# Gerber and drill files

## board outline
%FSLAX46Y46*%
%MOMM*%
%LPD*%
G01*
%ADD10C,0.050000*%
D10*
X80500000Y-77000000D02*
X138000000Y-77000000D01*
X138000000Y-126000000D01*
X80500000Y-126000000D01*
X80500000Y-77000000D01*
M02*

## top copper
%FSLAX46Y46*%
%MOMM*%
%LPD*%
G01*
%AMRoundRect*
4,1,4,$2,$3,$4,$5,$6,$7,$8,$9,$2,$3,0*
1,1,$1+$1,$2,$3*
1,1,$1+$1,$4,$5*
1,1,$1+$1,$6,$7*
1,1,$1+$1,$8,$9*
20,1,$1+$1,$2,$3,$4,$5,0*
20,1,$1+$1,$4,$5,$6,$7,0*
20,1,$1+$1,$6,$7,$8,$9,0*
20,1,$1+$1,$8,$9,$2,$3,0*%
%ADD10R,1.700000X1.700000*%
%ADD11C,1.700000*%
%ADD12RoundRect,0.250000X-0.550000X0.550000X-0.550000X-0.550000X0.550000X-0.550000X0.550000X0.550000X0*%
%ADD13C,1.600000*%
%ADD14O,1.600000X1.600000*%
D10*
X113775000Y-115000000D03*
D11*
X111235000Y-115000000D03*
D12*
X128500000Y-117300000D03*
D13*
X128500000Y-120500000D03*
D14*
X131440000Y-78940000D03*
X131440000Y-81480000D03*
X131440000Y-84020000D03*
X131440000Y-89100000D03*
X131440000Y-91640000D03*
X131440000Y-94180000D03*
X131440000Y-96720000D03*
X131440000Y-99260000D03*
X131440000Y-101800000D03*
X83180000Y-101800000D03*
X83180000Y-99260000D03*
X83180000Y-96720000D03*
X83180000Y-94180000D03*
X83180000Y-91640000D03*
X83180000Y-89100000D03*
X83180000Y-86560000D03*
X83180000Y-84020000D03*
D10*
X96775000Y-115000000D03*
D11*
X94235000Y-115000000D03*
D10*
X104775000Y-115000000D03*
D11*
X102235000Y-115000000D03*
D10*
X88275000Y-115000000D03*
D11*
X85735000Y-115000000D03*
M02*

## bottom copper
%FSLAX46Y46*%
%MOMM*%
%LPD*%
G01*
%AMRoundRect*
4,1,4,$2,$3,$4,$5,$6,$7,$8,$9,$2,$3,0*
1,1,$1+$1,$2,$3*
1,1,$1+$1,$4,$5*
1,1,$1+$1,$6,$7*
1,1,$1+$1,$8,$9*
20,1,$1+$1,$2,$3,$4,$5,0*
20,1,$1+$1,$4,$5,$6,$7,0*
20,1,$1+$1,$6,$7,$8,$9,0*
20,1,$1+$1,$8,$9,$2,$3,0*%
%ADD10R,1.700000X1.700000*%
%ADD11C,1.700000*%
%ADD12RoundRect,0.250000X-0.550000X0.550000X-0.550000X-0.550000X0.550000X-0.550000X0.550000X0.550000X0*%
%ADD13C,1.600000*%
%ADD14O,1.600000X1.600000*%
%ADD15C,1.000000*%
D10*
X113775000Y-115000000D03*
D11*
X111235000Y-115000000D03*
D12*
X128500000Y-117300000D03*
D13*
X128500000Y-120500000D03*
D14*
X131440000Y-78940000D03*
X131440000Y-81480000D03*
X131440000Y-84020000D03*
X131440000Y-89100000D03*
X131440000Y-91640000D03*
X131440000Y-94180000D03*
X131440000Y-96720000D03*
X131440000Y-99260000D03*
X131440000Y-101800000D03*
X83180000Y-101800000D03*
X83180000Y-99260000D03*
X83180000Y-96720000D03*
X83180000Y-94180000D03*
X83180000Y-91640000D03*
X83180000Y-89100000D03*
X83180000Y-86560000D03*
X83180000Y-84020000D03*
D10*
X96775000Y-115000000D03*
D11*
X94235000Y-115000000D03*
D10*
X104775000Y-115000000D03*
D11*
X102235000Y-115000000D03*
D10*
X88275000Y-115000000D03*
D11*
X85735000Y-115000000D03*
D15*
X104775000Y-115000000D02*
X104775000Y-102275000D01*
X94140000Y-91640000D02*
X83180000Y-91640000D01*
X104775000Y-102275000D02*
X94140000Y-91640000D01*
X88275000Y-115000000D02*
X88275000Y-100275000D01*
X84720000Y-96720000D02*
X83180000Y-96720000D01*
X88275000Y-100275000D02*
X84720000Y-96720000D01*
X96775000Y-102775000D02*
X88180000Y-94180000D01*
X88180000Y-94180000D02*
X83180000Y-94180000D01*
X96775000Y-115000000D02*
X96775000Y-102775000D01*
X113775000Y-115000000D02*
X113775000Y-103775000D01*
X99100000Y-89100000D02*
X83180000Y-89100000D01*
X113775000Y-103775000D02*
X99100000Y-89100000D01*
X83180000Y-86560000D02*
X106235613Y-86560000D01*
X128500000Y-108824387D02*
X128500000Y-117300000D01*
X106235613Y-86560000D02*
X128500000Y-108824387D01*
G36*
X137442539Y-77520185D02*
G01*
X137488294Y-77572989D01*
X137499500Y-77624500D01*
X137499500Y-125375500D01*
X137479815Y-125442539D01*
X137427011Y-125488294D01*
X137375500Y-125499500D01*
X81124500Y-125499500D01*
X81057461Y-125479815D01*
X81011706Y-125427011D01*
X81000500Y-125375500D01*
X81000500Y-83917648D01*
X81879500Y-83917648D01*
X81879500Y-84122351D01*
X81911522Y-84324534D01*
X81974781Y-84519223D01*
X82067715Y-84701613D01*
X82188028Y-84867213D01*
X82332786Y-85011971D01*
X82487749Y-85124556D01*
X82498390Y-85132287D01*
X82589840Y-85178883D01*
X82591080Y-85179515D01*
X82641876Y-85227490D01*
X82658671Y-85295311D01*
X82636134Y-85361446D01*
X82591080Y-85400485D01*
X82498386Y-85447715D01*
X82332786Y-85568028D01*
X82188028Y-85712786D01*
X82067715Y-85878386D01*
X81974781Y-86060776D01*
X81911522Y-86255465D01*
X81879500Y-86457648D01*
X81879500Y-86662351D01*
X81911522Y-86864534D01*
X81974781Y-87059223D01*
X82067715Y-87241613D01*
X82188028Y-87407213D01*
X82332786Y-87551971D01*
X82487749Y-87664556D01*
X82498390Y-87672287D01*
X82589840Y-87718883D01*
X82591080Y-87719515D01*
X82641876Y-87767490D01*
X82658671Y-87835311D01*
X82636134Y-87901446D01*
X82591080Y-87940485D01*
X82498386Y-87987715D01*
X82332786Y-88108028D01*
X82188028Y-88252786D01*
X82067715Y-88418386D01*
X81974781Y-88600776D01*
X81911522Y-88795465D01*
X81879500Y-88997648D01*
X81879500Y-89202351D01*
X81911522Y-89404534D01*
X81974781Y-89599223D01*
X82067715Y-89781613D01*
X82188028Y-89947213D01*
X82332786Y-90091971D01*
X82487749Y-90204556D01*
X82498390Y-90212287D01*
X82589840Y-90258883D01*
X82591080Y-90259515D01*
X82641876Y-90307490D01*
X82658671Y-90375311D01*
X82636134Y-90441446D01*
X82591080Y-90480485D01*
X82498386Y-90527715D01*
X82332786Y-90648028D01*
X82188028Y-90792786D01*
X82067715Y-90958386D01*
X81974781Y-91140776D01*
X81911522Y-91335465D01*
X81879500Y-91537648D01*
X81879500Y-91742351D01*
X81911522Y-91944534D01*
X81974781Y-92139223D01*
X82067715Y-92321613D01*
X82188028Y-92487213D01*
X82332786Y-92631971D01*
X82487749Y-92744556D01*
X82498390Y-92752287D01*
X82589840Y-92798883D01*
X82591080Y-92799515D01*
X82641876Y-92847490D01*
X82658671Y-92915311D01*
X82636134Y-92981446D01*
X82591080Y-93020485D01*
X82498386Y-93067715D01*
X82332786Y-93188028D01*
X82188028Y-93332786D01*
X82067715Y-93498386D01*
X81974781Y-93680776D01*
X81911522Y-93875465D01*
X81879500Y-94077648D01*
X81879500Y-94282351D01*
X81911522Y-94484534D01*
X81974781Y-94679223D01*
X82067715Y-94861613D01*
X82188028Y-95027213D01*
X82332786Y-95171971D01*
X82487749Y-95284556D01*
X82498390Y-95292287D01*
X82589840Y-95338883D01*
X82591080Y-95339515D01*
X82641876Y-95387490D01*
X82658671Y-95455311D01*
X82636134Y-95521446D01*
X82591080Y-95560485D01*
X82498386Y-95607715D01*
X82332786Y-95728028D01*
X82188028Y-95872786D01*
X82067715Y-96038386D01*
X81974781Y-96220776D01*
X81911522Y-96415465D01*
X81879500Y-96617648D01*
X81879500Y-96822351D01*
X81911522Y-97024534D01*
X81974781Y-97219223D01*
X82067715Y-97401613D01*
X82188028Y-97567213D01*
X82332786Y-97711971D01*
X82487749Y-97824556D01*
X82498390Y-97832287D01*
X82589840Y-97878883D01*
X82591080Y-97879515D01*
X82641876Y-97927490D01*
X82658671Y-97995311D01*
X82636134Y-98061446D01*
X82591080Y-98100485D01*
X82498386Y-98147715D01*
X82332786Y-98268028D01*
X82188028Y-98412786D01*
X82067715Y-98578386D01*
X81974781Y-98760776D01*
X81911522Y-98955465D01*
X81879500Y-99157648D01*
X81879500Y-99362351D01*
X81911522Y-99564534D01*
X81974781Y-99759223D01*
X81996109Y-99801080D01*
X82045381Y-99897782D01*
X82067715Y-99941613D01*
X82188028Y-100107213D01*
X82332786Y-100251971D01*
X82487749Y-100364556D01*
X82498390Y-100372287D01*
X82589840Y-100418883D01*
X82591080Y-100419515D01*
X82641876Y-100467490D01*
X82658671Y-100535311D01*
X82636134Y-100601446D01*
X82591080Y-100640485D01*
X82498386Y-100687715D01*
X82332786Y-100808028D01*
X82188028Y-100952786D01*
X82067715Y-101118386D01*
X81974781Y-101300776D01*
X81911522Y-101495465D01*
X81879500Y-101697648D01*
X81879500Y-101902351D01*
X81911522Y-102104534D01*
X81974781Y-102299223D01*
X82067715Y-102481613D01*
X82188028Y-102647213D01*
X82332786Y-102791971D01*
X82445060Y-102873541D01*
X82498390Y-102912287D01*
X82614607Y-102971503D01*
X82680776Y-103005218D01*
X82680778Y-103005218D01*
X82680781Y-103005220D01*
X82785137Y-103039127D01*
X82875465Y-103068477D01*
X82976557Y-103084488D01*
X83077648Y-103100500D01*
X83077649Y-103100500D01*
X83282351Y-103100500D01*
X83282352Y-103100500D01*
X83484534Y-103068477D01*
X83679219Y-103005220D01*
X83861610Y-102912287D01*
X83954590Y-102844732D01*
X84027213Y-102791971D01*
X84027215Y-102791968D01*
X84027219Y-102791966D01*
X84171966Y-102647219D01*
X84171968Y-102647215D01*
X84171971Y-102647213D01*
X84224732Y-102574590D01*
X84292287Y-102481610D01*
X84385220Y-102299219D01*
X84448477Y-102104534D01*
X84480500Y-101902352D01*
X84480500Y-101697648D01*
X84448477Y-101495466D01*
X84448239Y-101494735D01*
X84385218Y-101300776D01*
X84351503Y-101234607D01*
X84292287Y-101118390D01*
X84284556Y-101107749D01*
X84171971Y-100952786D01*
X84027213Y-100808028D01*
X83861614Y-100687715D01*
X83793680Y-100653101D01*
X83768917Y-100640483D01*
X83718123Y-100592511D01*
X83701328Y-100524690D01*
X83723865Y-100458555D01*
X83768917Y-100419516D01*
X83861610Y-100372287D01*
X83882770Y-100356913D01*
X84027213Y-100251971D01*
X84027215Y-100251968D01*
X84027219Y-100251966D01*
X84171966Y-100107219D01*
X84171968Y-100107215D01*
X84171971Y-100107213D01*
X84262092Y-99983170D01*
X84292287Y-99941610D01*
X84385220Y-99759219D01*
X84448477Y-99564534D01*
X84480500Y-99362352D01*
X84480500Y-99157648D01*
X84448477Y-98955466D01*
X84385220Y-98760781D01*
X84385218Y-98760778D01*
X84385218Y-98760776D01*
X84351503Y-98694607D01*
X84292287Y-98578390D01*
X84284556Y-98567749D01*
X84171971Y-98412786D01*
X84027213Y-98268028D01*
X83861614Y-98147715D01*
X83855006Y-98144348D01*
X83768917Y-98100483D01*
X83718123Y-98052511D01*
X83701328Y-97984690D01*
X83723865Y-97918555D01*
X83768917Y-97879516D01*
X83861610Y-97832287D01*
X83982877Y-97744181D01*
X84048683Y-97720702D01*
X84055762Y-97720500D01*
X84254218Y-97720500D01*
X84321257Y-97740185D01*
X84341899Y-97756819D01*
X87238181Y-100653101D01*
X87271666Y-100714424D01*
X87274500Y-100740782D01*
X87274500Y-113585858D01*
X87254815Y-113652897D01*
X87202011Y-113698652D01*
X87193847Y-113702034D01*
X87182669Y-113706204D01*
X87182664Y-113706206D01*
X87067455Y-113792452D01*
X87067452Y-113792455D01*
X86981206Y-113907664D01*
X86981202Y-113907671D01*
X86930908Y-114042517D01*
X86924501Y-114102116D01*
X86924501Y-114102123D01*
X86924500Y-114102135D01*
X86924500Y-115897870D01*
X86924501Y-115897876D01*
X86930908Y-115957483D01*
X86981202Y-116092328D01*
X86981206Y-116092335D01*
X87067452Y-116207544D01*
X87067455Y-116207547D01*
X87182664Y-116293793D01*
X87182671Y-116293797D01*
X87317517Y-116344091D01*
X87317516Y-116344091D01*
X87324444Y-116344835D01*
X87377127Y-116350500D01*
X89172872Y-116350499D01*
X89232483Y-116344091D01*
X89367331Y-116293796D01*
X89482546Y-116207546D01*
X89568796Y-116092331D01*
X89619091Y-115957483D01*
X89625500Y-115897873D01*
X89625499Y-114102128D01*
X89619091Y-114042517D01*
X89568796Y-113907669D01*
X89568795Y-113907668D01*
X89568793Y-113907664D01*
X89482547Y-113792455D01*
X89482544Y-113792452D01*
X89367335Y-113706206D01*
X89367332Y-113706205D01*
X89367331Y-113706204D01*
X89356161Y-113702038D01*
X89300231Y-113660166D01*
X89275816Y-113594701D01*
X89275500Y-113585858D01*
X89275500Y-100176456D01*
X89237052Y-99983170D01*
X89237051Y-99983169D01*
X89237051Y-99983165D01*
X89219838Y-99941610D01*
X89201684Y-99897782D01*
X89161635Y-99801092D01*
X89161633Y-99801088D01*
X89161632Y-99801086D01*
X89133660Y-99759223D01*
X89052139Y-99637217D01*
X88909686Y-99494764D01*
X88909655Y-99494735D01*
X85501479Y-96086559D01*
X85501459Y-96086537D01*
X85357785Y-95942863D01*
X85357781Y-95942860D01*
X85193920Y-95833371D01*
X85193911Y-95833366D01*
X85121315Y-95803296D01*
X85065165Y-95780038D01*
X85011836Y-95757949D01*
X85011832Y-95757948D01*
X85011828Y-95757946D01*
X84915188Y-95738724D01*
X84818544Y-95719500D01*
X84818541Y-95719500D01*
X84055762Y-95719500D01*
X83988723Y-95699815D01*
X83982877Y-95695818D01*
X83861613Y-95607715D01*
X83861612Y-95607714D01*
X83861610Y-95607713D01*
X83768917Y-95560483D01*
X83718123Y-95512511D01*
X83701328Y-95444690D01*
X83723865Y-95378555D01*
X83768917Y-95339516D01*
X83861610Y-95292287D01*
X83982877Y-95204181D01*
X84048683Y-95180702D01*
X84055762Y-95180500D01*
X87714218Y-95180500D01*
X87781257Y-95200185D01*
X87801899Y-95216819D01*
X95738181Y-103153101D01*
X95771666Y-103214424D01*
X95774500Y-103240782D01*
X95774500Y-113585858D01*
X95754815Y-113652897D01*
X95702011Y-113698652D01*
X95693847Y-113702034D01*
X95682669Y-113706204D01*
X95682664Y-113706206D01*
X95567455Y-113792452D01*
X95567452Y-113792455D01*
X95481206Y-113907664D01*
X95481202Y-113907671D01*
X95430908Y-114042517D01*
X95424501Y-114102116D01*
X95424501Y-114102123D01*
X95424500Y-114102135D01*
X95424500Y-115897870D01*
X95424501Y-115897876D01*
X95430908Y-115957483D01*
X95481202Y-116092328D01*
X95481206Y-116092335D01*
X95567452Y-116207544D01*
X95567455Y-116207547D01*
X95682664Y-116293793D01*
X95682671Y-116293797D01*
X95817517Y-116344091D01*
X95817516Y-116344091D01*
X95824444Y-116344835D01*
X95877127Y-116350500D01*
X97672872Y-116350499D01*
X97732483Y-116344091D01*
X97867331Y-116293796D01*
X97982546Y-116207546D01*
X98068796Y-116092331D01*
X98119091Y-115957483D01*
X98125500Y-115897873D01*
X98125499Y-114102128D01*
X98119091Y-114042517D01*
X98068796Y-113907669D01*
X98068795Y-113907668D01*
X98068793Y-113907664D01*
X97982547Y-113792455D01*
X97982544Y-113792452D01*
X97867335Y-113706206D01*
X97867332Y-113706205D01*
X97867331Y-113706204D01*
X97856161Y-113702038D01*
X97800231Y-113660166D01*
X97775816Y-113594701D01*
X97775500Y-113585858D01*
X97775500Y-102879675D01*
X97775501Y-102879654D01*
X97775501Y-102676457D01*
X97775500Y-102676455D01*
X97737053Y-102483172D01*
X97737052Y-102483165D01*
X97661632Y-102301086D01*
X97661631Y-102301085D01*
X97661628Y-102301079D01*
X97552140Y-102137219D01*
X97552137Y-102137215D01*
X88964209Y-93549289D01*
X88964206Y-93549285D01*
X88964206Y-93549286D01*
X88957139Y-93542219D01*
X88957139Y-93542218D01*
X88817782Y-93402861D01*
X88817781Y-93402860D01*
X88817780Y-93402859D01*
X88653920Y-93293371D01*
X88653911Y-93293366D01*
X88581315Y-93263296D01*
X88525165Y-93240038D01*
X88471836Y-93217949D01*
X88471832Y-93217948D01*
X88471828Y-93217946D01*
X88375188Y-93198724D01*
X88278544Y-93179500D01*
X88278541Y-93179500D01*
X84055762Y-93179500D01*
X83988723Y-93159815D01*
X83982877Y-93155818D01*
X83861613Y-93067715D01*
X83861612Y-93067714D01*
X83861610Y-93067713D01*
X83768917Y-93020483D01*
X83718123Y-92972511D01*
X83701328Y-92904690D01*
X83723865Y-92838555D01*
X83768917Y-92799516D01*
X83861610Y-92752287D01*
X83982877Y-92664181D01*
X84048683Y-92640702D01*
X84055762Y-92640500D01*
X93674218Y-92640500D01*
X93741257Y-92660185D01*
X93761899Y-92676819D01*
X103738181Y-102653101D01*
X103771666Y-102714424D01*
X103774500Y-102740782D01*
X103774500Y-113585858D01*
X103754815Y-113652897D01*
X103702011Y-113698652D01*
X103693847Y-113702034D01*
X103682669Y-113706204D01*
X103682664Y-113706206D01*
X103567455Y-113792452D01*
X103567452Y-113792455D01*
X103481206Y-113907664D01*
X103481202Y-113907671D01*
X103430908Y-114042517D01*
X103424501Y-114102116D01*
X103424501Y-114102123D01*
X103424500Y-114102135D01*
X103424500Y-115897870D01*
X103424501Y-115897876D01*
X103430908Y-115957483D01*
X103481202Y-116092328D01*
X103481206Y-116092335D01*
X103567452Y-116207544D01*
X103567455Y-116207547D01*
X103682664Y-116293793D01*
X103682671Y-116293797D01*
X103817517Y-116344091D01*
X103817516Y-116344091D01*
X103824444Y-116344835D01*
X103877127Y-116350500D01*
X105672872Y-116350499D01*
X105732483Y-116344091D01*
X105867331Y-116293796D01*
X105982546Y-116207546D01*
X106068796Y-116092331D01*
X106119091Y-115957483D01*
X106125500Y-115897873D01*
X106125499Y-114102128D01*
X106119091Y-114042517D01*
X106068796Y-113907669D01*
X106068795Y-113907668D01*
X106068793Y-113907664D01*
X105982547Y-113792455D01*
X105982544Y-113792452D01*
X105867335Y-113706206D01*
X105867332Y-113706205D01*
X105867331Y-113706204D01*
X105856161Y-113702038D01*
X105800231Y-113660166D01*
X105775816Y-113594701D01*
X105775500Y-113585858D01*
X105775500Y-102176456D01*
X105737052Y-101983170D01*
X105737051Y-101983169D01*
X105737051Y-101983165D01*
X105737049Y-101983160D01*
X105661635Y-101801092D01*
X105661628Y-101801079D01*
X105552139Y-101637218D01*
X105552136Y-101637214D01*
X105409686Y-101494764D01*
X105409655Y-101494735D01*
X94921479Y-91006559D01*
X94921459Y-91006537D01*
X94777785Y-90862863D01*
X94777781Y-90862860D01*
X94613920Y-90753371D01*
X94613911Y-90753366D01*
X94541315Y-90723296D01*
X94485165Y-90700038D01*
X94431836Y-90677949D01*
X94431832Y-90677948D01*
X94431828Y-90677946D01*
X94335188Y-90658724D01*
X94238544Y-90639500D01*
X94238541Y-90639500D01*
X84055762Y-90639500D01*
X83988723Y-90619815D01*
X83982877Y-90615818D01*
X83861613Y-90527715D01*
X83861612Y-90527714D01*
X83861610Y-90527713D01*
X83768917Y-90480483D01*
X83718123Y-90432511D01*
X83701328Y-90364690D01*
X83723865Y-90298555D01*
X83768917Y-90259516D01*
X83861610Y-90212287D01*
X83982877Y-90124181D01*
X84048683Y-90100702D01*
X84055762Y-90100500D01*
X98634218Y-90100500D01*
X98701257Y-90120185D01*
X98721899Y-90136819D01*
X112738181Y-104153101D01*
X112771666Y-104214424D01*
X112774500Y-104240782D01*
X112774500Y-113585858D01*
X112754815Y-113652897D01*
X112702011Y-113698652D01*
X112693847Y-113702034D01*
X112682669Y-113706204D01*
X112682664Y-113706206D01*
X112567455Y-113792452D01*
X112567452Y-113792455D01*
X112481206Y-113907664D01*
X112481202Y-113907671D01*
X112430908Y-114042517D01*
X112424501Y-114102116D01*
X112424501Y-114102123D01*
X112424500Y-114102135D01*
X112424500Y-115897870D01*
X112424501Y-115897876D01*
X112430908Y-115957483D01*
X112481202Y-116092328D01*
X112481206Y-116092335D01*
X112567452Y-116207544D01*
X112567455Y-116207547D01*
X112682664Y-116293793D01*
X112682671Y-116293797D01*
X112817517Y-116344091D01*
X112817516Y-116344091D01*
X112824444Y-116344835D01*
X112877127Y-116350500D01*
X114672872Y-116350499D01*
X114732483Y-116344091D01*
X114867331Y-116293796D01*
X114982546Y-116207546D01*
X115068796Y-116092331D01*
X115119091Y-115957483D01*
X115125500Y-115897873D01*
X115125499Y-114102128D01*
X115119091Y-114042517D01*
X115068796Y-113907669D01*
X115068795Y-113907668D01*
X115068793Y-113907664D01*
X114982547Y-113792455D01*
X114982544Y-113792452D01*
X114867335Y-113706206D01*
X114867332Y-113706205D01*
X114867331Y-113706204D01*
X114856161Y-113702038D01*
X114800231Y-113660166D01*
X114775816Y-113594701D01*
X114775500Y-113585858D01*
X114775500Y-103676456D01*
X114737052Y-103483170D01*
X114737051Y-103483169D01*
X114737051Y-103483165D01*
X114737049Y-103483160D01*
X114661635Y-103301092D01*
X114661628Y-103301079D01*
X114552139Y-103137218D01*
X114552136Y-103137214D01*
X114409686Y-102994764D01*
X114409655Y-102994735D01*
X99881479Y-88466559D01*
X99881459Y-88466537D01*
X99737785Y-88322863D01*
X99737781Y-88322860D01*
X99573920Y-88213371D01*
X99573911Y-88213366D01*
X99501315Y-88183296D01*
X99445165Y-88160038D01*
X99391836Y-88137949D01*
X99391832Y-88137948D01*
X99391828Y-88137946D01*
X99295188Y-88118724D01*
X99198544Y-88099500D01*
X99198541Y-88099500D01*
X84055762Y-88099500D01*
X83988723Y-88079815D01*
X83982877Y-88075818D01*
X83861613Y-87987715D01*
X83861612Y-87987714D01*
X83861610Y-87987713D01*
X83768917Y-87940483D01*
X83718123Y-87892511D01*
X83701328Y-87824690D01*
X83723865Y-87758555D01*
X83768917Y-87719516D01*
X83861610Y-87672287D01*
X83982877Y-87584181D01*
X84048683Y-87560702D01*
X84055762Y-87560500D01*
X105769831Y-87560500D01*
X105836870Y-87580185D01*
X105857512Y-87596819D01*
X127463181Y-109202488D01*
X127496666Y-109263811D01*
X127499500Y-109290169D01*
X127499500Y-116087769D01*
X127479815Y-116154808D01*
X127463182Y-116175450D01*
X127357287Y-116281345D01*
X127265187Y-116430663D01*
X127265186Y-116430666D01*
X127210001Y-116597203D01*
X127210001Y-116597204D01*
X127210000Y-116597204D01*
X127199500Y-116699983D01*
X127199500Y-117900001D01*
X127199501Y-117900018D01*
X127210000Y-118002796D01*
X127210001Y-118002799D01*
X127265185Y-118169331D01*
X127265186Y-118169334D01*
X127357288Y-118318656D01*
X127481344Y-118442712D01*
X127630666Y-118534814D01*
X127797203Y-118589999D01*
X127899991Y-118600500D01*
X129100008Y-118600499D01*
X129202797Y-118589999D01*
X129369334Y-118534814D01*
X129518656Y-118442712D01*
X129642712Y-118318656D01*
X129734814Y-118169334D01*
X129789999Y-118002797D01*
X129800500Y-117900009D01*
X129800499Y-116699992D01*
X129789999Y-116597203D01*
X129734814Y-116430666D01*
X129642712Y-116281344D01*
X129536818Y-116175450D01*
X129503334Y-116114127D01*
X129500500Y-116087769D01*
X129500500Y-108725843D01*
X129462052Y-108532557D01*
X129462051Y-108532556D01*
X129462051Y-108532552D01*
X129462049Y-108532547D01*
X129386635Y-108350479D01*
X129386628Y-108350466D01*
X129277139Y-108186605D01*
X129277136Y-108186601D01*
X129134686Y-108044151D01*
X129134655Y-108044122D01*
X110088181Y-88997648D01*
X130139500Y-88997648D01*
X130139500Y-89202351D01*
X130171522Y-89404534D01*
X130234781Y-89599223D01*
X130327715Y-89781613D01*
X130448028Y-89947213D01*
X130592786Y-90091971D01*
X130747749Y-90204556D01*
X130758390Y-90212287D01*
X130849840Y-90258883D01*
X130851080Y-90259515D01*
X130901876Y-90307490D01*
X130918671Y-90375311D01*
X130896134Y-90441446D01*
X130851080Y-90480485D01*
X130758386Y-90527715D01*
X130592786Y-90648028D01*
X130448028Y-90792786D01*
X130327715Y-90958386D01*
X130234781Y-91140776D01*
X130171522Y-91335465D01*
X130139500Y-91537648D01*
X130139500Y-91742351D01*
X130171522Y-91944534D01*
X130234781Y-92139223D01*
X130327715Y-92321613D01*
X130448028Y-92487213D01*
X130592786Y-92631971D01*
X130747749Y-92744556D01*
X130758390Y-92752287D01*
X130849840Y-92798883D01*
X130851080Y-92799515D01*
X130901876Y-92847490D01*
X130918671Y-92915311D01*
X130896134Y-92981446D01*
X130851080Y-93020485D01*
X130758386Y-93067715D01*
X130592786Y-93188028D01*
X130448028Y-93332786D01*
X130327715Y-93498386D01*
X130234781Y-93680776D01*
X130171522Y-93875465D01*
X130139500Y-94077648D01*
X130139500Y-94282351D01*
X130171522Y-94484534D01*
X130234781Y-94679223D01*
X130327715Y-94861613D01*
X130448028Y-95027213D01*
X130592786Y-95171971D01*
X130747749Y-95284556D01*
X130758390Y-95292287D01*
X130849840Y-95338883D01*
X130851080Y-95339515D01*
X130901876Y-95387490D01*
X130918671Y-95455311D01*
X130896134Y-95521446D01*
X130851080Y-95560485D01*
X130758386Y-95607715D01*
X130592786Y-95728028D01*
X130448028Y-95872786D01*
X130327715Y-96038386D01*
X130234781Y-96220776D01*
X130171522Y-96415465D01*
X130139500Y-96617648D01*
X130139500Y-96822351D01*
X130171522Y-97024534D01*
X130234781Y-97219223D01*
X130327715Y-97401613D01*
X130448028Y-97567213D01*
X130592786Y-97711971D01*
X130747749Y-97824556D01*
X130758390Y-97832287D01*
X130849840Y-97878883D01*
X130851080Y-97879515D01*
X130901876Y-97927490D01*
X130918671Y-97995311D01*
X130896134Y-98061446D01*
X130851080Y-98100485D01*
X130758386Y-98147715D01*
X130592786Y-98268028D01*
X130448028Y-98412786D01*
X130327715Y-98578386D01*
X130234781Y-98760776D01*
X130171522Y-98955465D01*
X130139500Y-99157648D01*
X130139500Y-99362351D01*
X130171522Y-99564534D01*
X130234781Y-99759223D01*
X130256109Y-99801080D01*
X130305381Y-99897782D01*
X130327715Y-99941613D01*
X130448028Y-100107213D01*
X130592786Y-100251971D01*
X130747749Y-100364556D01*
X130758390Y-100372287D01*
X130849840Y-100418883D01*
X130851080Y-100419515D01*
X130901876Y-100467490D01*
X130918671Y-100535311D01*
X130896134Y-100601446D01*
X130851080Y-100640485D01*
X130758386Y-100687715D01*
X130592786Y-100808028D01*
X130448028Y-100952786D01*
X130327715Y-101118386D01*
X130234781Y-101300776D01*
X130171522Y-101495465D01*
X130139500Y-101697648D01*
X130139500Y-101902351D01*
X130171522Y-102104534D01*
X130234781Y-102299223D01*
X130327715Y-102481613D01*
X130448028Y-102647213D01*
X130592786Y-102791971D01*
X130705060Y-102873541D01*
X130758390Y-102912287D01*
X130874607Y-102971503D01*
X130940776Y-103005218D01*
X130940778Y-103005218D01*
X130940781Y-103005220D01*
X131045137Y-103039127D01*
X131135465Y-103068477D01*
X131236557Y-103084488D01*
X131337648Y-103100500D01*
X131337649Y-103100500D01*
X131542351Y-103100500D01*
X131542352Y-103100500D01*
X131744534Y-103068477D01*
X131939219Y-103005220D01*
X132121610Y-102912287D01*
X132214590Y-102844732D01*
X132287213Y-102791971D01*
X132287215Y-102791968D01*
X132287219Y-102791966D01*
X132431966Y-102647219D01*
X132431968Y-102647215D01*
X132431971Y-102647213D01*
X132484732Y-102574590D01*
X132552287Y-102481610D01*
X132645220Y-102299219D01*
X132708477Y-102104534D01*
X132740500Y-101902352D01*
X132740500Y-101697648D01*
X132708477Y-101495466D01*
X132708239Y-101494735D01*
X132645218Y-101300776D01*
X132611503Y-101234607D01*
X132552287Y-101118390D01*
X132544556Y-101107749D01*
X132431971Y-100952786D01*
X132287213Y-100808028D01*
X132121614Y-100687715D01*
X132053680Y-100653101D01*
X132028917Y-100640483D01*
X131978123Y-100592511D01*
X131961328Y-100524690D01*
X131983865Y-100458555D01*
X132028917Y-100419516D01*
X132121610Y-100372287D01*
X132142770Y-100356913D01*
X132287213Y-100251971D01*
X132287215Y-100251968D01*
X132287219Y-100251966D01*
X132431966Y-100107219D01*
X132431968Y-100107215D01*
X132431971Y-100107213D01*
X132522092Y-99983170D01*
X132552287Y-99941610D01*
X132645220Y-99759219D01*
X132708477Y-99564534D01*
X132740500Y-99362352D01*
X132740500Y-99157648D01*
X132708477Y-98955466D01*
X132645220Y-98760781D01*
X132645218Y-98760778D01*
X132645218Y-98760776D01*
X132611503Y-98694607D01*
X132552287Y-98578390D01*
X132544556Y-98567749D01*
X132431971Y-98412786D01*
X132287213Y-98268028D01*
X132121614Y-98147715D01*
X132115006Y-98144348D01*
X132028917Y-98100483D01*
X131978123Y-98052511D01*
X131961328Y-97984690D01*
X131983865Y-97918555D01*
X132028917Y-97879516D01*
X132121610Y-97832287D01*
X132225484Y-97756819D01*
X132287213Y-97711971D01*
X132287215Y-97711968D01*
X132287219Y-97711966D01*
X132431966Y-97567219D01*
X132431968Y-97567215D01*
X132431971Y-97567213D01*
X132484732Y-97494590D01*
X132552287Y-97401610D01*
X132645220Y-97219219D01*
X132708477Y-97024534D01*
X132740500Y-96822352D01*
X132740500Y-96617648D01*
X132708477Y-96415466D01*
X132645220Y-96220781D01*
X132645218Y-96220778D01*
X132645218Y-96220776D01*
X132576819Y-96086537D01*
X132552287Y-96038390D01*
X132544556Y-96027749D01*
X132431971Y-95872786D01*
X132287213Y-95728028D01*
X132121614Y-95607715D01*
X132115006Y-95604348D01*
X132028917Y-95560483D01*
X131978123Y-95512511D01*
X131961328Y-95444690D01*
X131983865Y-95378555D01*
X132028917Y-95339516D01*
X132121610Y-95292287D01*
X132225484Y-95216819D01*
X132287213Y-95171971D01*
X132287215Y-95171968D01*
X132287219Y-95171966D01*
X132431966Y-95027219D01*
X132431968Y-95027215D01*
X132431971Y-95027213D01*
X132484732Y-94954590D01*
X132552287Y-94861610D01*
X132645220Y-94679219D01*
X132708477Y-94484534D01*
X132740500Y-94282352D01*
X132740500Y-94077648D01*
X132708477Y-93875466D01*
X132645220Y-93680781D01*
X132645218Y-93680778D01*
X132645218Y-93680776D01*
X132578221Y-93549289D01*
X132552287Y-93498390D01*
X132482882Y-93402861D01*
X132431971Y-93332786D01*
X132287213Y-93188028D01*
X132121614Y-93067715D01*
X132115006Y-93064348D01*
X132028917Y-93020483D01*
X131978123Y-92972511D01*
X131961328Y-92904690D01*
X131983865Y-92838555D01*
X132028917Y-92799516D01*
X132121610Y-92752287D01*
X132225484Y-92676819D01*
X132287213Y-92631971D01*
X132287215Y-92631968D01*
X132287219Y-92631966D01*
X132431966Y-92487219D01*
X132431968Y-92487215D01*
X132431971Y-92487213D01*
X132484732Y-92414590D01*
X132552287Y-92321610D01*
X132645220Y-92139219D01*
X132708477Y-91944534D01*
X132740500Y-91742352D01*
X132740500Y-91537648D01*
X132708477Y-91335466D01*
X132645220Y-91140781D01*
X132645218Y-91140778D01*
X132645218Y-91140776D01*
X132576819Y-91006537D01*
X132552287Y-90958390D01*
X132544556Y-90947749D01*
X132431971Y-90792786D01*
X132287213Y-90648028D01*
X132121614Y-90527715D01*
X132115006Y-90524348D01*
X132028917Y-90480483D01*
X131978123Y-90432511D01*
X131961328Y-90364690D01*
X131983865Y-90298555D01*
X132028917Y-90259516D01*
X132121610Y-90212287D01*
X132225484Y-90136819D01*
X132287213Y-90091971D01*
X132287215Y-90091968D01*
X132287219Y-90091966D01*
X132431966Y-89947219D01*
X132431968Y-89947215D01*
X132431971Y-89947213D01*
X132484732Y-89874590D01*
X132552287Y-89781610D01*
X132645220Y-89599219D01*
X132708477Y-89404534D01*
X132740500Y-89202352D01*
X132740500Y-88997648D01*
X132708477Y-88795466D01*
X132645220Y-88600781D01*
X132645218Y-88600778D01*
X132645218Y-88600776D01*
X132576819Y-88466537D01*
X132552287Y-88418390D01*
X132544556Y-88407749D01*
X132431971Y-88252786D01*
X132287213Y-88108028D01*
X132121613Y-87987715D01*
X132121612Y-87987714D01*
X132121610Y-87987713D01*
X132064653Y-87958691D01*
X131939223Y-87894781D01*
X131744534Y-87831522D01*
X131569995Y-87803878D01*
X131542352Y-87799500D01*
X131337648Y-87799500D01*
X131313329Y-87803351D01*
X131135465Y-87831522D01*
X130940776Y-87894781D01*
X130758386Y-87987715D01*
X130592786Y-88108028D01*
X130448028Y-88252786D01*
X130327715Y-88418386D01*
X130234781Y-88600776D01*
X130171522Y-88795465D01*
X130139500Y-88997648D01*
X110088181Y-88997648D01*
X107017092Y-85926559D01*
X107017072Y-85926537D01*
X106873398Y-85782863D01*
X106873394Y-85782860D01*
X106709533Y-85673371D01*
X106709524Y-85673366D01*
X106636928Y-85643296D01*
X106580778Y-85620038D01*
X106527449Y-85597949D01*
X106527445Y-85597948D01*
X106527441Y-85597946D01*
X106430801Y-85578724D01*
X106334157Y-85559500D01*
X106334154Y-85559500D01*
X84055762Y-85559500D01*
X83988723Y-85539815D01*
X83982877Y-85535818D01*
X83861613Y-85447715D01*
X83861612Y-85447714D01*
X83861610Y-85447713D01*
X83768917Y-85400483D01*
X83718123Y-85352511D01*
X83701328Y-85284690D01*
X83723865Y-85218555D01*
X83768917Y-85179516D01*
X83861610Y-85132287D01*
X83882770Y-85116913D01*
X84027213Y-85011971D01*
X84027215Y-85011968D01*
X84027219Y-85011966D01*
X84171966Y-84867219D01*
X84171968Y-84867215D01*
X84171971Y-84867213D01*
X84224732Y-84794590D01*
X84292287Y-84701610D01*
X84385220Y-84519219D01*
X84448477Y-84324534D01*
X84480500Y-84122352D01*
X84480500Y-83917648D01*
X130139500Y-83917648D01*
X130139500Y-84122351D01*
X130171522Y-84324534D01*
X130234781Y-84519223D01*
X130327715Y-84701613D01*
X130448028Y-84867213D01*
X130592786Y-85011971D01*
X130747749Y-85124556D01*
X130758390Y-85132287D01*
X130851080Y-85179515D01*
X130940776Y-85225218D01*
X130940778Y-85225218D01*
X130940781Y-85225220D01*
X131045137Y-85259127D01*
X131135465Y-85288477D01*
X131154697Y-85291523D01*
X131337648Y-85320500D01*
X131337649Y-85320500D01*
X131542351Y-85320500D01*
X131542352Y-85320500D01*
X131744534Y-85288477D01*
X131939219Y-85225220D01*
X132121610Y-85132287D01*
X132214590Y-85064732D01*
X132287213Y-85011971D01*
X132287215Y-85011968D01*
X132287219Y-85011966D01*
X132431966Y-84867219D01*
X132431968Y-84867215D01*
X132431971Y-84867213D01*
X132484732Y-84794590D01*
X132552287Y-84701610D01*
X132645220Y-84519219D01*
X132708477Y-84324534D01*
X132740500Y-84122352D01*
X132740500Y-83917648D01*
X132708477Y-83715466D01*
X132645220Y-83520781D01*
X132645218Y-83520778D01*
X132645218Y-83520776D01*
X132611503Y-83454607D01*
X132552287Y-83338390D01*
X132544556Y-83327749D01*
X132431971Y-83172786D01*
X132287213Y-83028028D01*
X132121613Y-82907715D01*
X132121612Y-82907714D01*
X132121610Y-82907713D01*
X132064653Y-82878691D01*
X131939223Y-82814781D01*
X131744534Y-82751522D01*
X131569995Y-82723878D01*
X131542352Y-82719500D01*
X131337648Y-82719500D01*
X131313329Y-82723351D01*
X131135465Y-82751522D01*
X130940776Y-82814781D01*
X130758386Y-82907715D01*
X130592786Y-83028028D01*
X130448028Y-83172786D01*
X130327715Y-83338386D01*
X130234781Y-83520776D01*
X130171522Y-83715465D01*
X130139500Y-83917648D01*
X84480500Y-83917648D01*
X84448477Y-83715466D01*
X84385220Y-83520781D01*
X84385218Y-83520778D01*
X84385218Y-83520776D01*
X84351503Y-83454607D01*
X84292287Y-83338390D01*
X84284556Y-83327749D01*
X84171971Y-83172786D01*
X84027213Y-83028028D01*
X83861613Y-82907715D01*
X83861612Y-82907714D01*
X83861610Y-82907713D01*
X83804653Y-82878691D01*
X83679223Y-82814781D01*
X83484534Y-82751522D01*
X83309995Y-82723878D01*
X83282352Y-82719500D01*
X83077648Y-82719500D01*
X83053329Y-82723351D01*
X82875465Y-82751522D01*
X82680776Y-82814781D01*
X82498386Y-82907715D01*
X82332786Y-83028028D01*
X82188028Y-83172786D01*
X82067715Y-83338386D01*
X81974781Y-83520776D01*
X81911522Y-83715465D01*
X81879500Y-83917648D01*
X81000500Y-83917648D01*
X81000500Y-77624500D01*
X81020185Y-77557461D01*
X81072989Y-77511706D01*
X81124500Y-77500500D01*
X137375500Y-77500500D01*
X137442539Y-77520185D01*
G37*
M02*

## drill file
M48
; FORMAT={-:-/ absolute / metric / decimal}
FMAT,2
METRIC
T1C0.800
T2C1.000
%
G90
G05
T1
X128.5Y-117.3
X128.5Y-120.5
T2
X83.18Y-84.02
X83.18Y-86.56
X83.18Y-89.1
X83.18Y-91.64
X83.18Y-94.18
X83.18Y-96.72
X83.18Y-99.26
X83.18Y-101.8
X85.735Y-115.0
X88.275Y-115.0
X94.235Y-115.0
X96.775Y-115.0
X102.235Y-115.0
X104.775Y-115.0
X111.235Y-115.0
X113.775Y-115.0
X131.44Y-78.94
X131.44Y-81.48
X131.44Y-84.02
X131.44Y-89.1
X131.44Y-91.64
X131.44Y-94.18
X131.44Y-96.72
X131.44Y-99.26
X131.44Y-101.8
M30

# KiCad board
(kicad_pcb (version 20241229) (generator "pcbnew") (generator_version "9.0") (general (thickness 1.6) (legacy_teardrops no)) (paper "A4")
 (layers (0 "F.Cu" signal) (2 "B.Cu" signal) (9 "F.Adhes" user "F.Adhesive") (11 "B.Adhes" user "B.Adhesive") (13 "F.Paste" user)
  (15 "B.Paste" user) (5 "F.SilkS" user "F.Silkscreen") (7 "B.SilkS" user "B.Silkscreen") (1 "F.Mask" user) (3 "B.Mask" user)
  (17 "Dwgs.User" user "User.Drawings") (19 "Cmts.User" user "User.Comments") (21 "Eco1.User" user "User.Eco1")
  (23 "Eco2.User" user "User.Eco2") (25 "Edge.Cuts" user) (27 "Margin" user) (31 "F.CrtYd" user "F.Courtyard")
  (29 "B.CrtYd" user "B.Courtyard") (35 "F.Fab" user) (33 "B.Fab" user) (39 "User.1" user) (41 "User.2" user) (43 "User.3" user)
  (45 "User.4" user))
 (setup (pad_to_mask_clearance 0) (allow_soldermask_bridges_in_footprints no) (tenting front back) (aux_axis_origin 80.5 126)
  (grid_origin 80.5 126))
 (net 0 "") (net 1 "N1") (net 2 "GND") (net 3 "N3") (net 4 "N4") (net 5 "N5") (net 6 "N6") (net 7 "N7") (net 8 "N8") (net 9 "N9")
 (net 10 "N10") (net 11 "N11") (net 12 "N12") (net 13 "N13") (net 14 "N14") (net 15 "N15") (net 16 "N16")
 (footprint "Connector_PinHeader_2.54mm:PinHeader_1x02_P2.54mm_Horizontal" (layer "F.Cu") (at 113.775 115 -90)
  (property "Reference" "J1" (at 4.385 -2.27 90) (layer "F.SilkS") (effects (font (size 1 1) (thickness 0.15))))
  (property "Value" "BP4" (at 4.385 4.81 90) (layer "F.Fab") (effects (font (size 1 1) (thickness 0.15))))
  (pad "1" thru_hole rect (at 0 0 270) (size 1.7 1.7) (drill 1) (layers "*.Cu" "*.Mask") (remove_unused_layers no) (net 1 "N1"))
  (pad "2" thru_hole circle (at 0 2.54 270) (size 1.7 1.7) (drill 1) (layers "*.Cu" "*.Mask") (remove_unused_layers no) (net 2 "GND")))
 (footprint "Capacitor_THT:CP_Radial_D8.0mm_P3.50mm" (layer "F.Cu") (at 128.5 117 -90)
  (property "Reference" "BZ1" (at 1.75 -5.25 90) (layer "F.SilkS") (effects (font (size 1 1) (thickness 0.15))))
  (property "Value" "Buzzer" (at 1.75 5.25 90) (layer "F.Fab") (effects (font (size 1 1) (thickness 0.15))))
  (pad "1" thru_hole roundrect (at 0.3 0 270) (size 1.6 1.6) (drill 0.8) (layers "*.Cu" "*.Mask") (remove_unused_layers no)
   (roundrect_rratio 0.15625) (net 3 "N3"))
  (pad "2" thru_hole circle (at 3.5 0 270) (size 1.6 1.6) (drill 0.8) (layers "*.Cu" "*.Mask") (remove_unused_layers no) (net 2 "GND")))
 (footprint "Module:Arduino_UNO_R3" (layer "F.Cu") (at 131.44 66.24 -90)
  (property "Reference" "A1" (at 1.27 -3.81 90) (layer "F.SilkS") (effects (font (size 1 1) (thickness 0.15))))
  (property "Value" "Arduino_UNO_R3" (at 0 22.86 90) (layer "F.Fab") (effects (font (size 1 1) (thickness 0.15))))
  (pad "6" thru_hole oval (at 12.7 0) (size 1.6 1.6) (drill 1) (layers "*.Cu" "*.Mask") (remove_unused_layers no) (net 2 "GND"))
  (pad "7" thru_hole oval (at 15.24 0) (size 1.6 1.6) (drill 1) (layers "*.Cu" "*.Mask") (remove_unused_layers no) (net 2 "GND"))
  (pad "8" thru_hole oval (at 17.78 0) (size 1.6 1.6) (drill 1) (layers "*.Cu" "*.Mask") (remove_unused_layers no) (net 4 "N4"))
  (pad "9" thru_hole oval (at 22.86 0) (size 1.6 1.6) (drill 1) (layers "*.Cu" "*.Mask") (remove_unused_layers no) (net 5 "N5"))
  (pad "10" thru_hole oval (at 25.4 0) (size 1.6 1.6) (drill 1) (layers "*.Cu" "*.Mask") (remove_unused_layers no) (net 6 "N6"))
  (pad "11" thru_hole oval (at 27.94 0) (size 1.6 1.6) (drill 1) (layers "*.Cu" "*.Mask") (remove_unused_layers no) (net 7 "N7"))
  (pad "12" thru_hole oval (at 30.48 0) (size 1.6 1.6) (drill 1) (layers "*.Cu" "*.Mask") (remove_unused_layers no) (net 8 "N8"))
  (pad "13" thru_hole oval (at 33.02 0) (size 1.6 1.6) (drill 1) (layers "*.Cu" "*.Mask") (remove_unused_layers no) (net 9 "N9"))
  (pad "14" thru_hole oval (at 35.56 0) (size 1.6 1.6) (drill 1) (layers "*.Cu" "*.Mask") (remove_unused_layers no) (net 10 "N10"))
  (pad "15" thru_hole oval (at 35.56 48.26) (size 1.6 1.6) (drill 1) (layers "*.Cu" "*.Mask") (remove_unused_layers no) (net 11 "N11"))
  (pad "16" thru_hole oval (at 33.02 48.26) (size 1.6 1.6) (drill 1) (layers "*.Cu" "*.Mask") (remove_unused_layers no) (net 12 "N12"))
  (pad "17" thru_hole oval (at 30.48 48.26) (size 1.6 1.6) (drill 1) (layers "*.Cu" "*.Mask") (remove_unused_layers no) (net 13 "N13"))
  (pad "18" thru_hole oval (at 27.94 48.26) (size 1.6 1.6) (drill 1) (layers "*.Cu" "*.Mask") (remove_unused_layers no) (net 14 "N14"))
  (pad "19" thru_hole oval (at 25.4 48.26) (size 1.6 1.6) (drill 1) (layers "*.Cu" "*.Mask") (remove_unused_layers no) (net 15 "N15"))
  (pad "20" thru_hole oval (at 22.86 48.26) (size 1.6 1.6) (drill 1) (layers "*.Cu" "*.Mask") (remove_unused_layers no) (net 1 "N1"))
  (pad "21" thru_hole oval (at 20.32 48.26) (size 1.6 1.6) (drill 1) (layers "*.Cu" "*.Mask") (remove_unused_layers no) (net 3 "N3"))
  (pad "22" thru_hole oval (at 17.78 48.26) (size 1.6 1.6) (drill 1) (layers "*.Cu" "*.Mask") (remove_unused_layers no) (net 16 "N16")))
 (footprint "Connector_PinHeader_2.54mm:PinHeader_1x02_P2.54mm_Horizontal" (layer "F.Cu") (at 96.775 115 -90)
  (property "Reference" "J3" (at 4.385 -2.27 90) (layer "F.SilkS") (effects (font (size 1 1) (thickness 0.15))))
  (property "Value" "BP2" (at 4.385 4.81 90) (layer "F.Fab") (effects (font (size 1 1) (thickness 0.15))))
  (pad "1" thru_hole rect (at 0 0 270) (size 1.7 1.7) (drill 1) (layers "*.Cu" "*.Mask") (remove_unused_layers no) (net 14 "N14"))
  (pad "2" thru_hole circle (at 0 2.54 270) (size 1.7 1.7) (drill 1) (layers "*.Cu" "*.Mask") (remove_unused_layers no) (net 2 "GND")))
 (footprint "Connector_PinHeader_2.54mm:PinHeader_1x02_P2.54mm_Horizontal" (layer "F.Cu") (at 104.775 115 -90)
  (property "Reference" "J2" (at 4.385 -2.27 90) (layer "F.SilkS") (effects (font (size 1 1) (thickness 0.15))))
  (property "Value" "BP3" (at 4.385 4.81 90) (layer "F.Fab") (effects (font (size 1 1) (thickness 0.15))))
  (pad "1" thru_hole rect (at 0 0 270) (size 1.7 1.7) (drill 1) (layers "*.Cu" "*.Mask") (remove_unused_layers no) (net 15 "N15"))
  (pad "2" thru_hole circle (at 0 2.54 270) (size 1.7 1.7) (drill 1) (layers "*.Cu" "*.Mask") (remove_unused_layers no) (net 2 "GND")))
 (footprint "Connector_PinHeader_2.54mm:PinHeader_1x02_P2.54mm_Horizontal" (layer "F.Cu") (at 88.275 115 -90)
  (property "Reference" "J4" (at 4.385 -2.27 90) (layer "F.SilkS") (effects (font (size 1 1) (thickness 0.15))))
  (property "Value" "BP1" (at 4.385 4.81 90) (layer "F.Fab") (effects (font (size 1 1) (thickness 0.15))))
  (pad "1" thru_hole rect (at 0 0 270) (size 1.7 1.7) (drill 1) (layers "*.Cu" "*.Mask") (remove_unused_layers no) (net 13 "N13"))
  (pad "2" thru_hole circle (at 0 2.54 270) (size 1.7 1.7) (drill 1) (layers "*.Cu" "*.Mask") (remove_unused_layers no) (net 2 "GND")))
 (gr_rect (start 80.5 77) (end 138 126) (stroke (width 0.05) (type default)) (fill no) (layer "Edge.Cuts"))
 (segment (start 104.775 115) (end 104.775 102.275) (width 1) (layer "B.Cu") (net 15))
 (segment (start 94.14 91.64) (end 83.18 91.64) (width 1) (layer "B.Cu") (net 15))
 (segment (start 104.775 102.275) (end 94.14 91.64) (width 1) (layer "B.Cu") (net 15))
 (segment (start 88.275 115) (end 88.275 100.275) (width 1) (layer "B.Cu") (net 13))
 (segment (start 84.72 96.72) (end 83.18 96.72) (width 1) (layer "B.Cu") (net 13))
 (segment (start 88.275 100.275) (end 84.72 96.72) (width 1) (layer "B.Cu") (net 13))
 (segment (start 96.775 102.775) (end 88.18 94.18) (width 1) (layer "B.Cu") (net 14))
 (segment (start 88.18 94.18) (end 83.18 94.18) (width 1) (layer "B.Cu") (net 14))
 (segment (start 96.775 115) (end 96.775 102.775) (width 1) (layer "B.Cu") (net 14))
 (segment (start 113.775 115) (end 113.775 103.775) (width 1) (layer "B.Cu") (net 1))
 (segment (start 99.1 89.1) (end 83.18 89.1) (width 1) (layer "B.Cu") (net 1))
 (segment (start 113.775 103.775) (end 99.1 89.1) (width 1) (layer "B.Cu") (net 1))
 (segment (start 83.18 86.56) (end 106.235613 86.56) (width 1) (layer "B.Cu") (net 3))
 (segment (start 128.5 108.824387) (end 128.5 117.3) (width 1) (layer "B.Cu") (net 3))
 (segment (start 106.235613 86.56) (end 128.5 108.824387) (width 1) (layer "B.Cu") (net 3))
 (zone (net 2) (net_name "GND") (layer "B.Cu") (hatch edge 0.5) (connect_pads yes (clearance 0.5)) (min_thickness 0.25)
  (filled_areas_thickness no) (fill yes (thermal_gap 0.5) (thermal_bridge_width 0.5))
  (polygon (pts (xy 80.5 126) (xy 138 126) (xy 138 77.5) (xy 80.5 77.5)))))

